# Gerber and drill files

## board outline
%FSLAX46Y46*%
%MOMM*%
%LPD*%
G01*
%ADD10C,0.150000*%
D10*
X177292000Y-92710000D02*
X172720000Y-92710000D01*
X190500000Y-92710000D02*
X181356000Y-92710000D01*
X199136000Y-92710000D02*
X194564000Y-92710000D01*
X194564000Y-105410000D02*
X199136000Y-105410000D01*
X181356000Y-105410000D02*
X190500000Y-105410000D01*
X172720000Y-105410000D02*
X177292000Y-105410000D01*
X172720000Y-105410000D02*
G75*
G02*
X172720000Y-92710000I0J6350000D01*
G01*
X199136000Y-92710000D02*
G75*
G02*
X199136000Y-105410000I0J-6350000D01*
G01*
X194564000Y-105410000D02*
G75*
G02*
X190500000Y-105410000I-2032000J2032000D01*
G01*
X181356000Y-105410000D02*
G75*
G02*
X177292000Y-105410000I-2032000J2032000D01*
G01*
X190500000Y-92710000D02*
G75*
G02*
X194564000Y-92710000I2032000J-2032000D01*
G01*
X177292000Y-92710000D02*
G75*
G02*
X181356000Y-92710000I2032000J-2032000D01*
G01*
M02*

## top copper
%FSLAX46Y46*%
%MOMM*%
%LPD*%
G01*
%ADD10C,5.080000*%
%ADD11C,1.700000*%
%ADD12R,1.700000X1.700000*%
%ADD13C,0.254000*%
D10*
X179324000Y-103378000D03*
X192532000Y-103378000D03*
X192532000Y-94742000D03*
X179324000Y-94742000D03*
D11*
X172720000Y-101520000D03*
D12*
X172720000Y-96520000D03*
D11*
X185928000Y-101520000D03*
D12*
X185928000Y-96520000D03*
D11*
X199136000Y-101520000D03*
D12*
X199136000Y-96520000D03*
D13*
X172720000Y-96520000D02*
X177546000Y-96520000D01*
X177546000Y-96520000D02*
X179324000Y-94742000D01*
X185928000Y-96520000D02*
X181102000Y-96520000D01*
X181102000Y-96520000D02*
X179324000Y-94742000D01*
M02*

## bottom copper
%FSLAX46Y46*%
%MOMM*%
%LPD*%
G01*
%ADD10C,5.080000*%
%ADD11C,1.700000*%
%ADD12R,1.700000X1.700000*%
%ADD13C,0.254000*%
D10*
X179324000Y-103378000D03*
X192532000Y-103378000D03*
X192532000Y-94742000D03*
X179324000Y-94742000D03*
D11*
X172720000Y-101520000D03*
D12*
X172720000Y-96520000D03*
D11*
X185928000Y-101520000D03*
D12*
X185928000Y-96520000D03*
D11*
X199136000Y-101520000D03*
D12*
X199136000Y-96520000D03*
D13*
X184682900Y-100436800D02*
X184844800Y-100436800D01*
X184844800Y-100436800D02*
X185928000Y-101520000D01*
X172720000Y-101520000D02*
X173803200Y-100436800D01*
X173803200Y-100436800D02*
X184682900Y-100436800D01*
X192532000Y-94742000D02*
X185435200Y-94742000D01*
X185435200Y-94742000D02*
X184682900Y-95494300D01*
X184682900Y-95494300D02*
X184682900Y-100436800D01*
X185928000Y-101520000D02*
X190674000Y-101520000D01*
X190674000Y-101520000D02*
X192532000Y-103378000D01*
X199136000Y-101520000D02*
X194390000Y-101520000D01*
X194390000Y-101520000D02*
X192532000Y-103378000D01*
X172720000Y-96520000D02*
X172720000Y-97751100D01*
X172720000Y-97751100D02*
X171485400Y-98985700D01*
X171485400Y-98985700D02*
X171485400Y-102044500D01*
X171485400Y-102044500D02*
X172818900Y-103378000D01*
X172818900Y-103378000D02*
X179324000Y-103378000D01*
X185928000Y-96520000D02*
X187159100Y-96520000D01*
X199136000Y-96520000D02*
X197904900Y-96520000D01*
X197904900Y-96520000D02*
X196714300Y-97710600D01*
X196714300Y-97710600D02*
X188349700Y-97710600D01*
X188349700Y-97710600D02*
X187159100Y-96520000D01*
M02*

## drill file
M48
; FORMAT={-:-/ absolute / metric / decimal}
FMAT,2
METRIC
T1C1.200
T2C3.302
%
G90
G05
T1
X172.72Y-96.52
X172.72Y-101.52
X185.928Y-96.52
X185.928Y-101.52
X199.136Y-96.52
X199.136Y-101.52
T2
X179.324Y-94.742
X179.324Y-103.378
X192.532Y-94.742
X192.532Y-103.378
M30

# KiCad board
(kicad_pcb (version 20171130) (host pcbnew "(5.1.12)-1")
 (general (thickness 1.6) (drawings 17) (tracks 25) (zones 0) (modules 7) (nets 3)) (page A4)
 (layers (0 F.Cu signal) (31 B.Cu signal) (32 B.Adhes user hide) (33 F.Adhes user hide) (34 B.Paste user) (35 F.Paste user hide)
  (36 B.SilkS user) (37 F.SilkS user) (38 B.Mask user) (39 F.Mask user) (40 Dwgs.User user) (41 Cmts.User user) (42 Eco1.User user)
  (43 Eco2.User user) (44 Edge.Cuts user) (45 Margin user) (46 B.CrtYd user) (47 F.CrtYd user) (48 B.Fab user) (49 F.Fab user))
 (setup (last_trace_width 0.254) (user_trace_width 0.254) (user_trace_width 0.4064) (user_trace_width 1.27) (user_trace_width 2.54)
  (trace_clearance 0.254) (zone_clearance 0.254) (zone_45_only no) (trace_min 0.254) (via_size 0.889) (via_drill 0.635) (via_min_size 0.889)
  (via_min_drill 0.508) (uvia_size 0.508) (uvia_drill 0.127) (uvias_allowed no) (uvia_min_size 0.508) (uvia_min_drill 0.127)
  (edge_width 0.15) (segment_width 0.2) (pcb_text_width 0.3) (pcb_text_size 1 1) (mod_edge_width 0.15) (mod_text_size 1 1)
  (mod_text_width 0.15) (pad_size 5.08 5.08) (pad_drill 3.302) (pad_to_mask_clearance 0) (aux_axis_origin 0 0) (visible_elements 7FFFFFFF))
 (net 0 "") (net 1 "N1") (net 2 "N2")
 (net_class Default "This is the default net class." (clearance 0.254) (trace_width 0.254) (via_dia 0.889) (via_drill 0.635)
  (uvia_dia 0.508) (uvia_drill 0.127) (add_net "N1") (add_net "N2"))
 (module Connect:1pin (layer F.Cu) (at 179.324 103.378)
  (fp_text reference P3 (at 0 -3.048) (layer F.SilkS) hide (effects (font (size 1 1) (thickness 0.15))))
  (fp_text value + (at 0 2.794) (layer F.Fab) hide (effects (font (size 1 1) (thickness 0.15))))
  (pad 1 thru_hole circle (at 0 0) (size 5.08 5.08) (drill 3.302) (layers *.Cu *.Mask F.SilkS) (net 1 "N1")))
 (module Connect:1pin (layer F.Cu) (at 192.532 103.378 90)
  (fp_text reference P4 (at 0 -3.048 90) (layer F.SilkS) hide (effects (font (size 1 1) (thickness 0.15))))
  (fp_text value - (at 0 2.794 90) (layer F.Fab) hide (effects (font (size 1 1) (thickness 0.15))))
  (pad 1 thru_hole circle (at 0 0 90) (size 5.08 5.08) (drill 3.302) (layers *.Cu *.Mask F.SilkS) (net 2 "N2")))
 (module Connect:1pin (layer F.Cu) (at 192.532 94.742)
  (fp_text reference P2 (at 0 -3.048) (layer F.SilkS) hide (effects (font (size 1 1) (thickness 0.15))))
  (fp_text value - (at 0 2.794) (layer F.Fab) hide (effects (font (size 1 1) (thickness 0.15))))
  (pad 1 thru_hole circle (at 0 0) (size 5.08 5.08) (drill 3.302) (layers *.Cu *.Mask F.SilkS) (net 2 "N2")))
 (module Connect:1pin (layer F.Cu) (at 179.324 94.742)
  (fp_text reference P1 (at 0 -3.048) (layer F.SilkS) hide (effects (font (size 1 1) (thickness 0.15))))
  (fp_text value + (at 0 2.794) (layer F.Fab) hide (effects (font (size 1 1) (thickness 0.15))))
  (pad 1 thru_hole circle (at 0 0) (size 5.08 5.08) (drill 3.302) (layers *.Cu *.Mask F.SilkS) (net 1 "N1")))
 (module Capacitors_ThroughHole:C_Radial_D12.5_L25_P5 (layer F.Cu) (at 172.72 96.52 270)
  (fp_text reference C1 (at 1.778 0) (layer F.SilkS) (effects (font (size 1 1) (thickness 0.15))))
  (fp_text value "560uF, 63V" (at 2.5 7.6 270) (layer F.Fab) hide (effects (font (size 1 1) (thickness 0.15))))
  (pad 2 thru_hole circle (at 5 0 270) (size 1.7 1.7) (drill 1.2) (layers *.Cu *.Mask F.SilkS) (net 2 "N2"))
  (pad 1 thru_hole rect (at 0 0 270) (size 1.7 1.7) (drill 1.2) (layers *.Cu *.Mask F.SilkS) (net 1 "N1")))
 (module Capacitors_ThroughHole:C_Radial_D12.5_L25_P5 (layer F.Cu) (at 185.928 96.52 270)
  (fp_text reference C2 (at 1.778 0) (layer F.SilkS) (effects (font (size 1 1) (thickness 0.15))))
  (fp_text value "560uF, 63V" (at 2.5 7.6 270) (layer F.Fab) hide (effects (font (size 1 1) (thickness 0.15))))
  (pad 2 thru_hole circle (at 5 0 270) (size 1.7 1.7) (drill 1.2) (layers *.Cu *.Mask F.SilkS) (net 2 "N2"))
  (pad 1 thru_hole rect (at 0 0 270) (size 1.7 1.7) (drill 1.2) (layers *.Cu *.Mask F.SilkS) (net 1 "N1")))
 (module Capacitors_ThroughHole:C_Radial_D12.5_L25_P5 (layer F.Cu) (at 199.136 96.52 270)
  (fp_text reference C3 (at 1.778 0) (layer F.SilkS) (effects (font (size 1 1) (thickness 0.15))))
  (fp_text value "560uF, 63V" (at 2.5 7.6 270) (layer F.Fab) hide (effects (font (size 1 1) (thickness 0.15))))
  (pad 2 thru_hole circle (at 5 0 270) (size 1.7 1.7) (drill 1.2) (layers *.Cu *.Mask F.SilkS) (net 2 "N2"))
  (pad 1 thru_hole rect (at 0 0 270) (size 1.7 1.7) (drill 1.2) (layers *.Cu *.Mask F.SilkS) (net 1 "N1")))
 (gr_line (start 177.292 92.71) (end 172.72 92.71) (angle 90) (layer Edge.Cuts) (width 0.15))
 (gr_line (start 190.5 92.71) (end 181.356 92.71) (angle 90) (layer Edge.Cuts) (width 0.15))
 (gr_line (start 199.136 92.71) (end 194.564 92.71) (angle 90) (layer Edge.Cuts) (width 0.15))
 (gr_line (start 194.564 105.41) (end 199.136 105.41) (angle 90) (layer Edge.Cuts) (width 0.15))
 (gr_line (start 181.356 105.41) (end 190.5 105.41) (angle 90) (layer Edge.Cuts) (width 0.15))
 (gr_line (start 172.72 105.41) (end 177.292 105.41) (angle 90) (layer Edge.Cuts) (width 0.15))
 (gr_arc (start 172.72 99.06) (end 172.72 105.41) (angle 180) (layer Edge.Cuts) (width 0.15))
 (gr_arc (start 199.136 99.06) (end 199.136 92.71) (angle 180) (layer Edge.Cuts) (width 0.15))
 (gr_arc (start 192.532 103.378) (end 194.564 105.41) (angle 90) (layer Edge.Cuts) (width 0.15))
 (gr_arc (start 179.324 103.378) (end 181.356 105.41) (angle 90) (layer Edge.Cuts) (width 0.15))
 (gr_arc (start 192.532 94.742) (end 190.5 92.71) (angle 90) (layer Edge.Cuts) (width 0.15))
 (gr_arc (start 179.324 94.742) (end 177.292 92.71) (angle 90) (layer Edge.Cuts) (width 0.15))
 (segment (start 184.6829 100.4368) (end 184.8448 100.4368) (width 0.254) (layer B.Cu) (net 2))
 (segment (start 184.8448 100.4368) (end 185.928 101.52) (width 0.254) (layer B.Cu) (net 2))
 (segment (start 172.72 101.52) (end 173.8032 100.4368) (width 0.254) (layer B.Cu) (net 2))
 (segment (start 173.8032 100.4368) (end 184.6829 100.4368) (width 0.254) (layer B.Cu) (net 2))
 (segment (start 192.532 94.742) (end 185.4352 94.742) (width 0.254) (layer B.Cu) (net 2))
 (segment (start 185.4352 94.742) (end 184.6829 95.4943) (width 0.254) (layer B.Cu) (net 2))
 (segment (start 184.6829 95.4943) (end 184.6829 100.4368) (width 0.254) (layer B.Cu) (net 2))
 (segment (start 185.928 101.52) (end 190.674 101.52) (width 0.254) (layer B.Cu) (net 2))
 (segment (start 190.674 101.52) (end 192.532 103.378) (width 0.254) (layer B.Cu) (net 2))
 (segment (start 199.136 101.52) (end 194.39 101.52) (width 0.254) (layer B.Cu) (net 2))
 (segment (start 194.39 101.52) (end 192.532 103.378) (width 0.254) (layer B.Cu) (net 2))
 (segment (start 172.72 96.52) (end 172.72 97.7511) (width 0.254) (layer B.Cu) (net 1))
 (segment (start 172.72 97.7511) (end 171.4854 98.9857) (width 0.254) (layer B.Cu) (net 1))
 (segment (start 171.4854 98.9857) (end 171.4854 102.0445) (width 0.254) (layer B.Cu) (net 1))
 (segment (start 171.4854 102.0445) (end 172.8189 103.378) (width 0.254) (layer B.Cu) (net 1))
 (segment (start 172.8189 103.378) (end 179.324 103.378) (width 0.254) (layer B.Cu) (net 1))
 (segment (start 172.72 96.52) (end 177.546 96.52) (width 0.254) (layer F.Cu) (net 1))
 (segment (start 177.546 96.52) (end 179.324 94.742) (width 0.254) (layer F.Cu) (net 1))
 (segment (start 185.928 96.52) (end 181.102 96.52) (width 0.254) (layer F.Cu) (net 1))
 (segment (start 181.102 96.52) (end 179.324 94.742) (width 0.254) (layer F.Cu) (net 1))
 (segment (start 185.928 96.52) (end 187.1591 96.52) (width 0.254) (layer B.Cu) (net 1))
 (segment (start 199.136 96.52) (end 197.9049 96.52) (width 0.254) (layer B.Cu) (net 1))
 (segment (start 197.9049 96.52) (end 196.7143 97.7106) (width 0.254) (layer B.Cu) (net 1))
 (segment (start 196.7143 97.7106) (end 188.3497 97.7106) (width 0.254) (layer B.Cu) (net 1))
 (segment (start 188.3497 97.7106) (end 187.1591 96.52) (width 0.254) (layer B.Cu) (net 1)))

